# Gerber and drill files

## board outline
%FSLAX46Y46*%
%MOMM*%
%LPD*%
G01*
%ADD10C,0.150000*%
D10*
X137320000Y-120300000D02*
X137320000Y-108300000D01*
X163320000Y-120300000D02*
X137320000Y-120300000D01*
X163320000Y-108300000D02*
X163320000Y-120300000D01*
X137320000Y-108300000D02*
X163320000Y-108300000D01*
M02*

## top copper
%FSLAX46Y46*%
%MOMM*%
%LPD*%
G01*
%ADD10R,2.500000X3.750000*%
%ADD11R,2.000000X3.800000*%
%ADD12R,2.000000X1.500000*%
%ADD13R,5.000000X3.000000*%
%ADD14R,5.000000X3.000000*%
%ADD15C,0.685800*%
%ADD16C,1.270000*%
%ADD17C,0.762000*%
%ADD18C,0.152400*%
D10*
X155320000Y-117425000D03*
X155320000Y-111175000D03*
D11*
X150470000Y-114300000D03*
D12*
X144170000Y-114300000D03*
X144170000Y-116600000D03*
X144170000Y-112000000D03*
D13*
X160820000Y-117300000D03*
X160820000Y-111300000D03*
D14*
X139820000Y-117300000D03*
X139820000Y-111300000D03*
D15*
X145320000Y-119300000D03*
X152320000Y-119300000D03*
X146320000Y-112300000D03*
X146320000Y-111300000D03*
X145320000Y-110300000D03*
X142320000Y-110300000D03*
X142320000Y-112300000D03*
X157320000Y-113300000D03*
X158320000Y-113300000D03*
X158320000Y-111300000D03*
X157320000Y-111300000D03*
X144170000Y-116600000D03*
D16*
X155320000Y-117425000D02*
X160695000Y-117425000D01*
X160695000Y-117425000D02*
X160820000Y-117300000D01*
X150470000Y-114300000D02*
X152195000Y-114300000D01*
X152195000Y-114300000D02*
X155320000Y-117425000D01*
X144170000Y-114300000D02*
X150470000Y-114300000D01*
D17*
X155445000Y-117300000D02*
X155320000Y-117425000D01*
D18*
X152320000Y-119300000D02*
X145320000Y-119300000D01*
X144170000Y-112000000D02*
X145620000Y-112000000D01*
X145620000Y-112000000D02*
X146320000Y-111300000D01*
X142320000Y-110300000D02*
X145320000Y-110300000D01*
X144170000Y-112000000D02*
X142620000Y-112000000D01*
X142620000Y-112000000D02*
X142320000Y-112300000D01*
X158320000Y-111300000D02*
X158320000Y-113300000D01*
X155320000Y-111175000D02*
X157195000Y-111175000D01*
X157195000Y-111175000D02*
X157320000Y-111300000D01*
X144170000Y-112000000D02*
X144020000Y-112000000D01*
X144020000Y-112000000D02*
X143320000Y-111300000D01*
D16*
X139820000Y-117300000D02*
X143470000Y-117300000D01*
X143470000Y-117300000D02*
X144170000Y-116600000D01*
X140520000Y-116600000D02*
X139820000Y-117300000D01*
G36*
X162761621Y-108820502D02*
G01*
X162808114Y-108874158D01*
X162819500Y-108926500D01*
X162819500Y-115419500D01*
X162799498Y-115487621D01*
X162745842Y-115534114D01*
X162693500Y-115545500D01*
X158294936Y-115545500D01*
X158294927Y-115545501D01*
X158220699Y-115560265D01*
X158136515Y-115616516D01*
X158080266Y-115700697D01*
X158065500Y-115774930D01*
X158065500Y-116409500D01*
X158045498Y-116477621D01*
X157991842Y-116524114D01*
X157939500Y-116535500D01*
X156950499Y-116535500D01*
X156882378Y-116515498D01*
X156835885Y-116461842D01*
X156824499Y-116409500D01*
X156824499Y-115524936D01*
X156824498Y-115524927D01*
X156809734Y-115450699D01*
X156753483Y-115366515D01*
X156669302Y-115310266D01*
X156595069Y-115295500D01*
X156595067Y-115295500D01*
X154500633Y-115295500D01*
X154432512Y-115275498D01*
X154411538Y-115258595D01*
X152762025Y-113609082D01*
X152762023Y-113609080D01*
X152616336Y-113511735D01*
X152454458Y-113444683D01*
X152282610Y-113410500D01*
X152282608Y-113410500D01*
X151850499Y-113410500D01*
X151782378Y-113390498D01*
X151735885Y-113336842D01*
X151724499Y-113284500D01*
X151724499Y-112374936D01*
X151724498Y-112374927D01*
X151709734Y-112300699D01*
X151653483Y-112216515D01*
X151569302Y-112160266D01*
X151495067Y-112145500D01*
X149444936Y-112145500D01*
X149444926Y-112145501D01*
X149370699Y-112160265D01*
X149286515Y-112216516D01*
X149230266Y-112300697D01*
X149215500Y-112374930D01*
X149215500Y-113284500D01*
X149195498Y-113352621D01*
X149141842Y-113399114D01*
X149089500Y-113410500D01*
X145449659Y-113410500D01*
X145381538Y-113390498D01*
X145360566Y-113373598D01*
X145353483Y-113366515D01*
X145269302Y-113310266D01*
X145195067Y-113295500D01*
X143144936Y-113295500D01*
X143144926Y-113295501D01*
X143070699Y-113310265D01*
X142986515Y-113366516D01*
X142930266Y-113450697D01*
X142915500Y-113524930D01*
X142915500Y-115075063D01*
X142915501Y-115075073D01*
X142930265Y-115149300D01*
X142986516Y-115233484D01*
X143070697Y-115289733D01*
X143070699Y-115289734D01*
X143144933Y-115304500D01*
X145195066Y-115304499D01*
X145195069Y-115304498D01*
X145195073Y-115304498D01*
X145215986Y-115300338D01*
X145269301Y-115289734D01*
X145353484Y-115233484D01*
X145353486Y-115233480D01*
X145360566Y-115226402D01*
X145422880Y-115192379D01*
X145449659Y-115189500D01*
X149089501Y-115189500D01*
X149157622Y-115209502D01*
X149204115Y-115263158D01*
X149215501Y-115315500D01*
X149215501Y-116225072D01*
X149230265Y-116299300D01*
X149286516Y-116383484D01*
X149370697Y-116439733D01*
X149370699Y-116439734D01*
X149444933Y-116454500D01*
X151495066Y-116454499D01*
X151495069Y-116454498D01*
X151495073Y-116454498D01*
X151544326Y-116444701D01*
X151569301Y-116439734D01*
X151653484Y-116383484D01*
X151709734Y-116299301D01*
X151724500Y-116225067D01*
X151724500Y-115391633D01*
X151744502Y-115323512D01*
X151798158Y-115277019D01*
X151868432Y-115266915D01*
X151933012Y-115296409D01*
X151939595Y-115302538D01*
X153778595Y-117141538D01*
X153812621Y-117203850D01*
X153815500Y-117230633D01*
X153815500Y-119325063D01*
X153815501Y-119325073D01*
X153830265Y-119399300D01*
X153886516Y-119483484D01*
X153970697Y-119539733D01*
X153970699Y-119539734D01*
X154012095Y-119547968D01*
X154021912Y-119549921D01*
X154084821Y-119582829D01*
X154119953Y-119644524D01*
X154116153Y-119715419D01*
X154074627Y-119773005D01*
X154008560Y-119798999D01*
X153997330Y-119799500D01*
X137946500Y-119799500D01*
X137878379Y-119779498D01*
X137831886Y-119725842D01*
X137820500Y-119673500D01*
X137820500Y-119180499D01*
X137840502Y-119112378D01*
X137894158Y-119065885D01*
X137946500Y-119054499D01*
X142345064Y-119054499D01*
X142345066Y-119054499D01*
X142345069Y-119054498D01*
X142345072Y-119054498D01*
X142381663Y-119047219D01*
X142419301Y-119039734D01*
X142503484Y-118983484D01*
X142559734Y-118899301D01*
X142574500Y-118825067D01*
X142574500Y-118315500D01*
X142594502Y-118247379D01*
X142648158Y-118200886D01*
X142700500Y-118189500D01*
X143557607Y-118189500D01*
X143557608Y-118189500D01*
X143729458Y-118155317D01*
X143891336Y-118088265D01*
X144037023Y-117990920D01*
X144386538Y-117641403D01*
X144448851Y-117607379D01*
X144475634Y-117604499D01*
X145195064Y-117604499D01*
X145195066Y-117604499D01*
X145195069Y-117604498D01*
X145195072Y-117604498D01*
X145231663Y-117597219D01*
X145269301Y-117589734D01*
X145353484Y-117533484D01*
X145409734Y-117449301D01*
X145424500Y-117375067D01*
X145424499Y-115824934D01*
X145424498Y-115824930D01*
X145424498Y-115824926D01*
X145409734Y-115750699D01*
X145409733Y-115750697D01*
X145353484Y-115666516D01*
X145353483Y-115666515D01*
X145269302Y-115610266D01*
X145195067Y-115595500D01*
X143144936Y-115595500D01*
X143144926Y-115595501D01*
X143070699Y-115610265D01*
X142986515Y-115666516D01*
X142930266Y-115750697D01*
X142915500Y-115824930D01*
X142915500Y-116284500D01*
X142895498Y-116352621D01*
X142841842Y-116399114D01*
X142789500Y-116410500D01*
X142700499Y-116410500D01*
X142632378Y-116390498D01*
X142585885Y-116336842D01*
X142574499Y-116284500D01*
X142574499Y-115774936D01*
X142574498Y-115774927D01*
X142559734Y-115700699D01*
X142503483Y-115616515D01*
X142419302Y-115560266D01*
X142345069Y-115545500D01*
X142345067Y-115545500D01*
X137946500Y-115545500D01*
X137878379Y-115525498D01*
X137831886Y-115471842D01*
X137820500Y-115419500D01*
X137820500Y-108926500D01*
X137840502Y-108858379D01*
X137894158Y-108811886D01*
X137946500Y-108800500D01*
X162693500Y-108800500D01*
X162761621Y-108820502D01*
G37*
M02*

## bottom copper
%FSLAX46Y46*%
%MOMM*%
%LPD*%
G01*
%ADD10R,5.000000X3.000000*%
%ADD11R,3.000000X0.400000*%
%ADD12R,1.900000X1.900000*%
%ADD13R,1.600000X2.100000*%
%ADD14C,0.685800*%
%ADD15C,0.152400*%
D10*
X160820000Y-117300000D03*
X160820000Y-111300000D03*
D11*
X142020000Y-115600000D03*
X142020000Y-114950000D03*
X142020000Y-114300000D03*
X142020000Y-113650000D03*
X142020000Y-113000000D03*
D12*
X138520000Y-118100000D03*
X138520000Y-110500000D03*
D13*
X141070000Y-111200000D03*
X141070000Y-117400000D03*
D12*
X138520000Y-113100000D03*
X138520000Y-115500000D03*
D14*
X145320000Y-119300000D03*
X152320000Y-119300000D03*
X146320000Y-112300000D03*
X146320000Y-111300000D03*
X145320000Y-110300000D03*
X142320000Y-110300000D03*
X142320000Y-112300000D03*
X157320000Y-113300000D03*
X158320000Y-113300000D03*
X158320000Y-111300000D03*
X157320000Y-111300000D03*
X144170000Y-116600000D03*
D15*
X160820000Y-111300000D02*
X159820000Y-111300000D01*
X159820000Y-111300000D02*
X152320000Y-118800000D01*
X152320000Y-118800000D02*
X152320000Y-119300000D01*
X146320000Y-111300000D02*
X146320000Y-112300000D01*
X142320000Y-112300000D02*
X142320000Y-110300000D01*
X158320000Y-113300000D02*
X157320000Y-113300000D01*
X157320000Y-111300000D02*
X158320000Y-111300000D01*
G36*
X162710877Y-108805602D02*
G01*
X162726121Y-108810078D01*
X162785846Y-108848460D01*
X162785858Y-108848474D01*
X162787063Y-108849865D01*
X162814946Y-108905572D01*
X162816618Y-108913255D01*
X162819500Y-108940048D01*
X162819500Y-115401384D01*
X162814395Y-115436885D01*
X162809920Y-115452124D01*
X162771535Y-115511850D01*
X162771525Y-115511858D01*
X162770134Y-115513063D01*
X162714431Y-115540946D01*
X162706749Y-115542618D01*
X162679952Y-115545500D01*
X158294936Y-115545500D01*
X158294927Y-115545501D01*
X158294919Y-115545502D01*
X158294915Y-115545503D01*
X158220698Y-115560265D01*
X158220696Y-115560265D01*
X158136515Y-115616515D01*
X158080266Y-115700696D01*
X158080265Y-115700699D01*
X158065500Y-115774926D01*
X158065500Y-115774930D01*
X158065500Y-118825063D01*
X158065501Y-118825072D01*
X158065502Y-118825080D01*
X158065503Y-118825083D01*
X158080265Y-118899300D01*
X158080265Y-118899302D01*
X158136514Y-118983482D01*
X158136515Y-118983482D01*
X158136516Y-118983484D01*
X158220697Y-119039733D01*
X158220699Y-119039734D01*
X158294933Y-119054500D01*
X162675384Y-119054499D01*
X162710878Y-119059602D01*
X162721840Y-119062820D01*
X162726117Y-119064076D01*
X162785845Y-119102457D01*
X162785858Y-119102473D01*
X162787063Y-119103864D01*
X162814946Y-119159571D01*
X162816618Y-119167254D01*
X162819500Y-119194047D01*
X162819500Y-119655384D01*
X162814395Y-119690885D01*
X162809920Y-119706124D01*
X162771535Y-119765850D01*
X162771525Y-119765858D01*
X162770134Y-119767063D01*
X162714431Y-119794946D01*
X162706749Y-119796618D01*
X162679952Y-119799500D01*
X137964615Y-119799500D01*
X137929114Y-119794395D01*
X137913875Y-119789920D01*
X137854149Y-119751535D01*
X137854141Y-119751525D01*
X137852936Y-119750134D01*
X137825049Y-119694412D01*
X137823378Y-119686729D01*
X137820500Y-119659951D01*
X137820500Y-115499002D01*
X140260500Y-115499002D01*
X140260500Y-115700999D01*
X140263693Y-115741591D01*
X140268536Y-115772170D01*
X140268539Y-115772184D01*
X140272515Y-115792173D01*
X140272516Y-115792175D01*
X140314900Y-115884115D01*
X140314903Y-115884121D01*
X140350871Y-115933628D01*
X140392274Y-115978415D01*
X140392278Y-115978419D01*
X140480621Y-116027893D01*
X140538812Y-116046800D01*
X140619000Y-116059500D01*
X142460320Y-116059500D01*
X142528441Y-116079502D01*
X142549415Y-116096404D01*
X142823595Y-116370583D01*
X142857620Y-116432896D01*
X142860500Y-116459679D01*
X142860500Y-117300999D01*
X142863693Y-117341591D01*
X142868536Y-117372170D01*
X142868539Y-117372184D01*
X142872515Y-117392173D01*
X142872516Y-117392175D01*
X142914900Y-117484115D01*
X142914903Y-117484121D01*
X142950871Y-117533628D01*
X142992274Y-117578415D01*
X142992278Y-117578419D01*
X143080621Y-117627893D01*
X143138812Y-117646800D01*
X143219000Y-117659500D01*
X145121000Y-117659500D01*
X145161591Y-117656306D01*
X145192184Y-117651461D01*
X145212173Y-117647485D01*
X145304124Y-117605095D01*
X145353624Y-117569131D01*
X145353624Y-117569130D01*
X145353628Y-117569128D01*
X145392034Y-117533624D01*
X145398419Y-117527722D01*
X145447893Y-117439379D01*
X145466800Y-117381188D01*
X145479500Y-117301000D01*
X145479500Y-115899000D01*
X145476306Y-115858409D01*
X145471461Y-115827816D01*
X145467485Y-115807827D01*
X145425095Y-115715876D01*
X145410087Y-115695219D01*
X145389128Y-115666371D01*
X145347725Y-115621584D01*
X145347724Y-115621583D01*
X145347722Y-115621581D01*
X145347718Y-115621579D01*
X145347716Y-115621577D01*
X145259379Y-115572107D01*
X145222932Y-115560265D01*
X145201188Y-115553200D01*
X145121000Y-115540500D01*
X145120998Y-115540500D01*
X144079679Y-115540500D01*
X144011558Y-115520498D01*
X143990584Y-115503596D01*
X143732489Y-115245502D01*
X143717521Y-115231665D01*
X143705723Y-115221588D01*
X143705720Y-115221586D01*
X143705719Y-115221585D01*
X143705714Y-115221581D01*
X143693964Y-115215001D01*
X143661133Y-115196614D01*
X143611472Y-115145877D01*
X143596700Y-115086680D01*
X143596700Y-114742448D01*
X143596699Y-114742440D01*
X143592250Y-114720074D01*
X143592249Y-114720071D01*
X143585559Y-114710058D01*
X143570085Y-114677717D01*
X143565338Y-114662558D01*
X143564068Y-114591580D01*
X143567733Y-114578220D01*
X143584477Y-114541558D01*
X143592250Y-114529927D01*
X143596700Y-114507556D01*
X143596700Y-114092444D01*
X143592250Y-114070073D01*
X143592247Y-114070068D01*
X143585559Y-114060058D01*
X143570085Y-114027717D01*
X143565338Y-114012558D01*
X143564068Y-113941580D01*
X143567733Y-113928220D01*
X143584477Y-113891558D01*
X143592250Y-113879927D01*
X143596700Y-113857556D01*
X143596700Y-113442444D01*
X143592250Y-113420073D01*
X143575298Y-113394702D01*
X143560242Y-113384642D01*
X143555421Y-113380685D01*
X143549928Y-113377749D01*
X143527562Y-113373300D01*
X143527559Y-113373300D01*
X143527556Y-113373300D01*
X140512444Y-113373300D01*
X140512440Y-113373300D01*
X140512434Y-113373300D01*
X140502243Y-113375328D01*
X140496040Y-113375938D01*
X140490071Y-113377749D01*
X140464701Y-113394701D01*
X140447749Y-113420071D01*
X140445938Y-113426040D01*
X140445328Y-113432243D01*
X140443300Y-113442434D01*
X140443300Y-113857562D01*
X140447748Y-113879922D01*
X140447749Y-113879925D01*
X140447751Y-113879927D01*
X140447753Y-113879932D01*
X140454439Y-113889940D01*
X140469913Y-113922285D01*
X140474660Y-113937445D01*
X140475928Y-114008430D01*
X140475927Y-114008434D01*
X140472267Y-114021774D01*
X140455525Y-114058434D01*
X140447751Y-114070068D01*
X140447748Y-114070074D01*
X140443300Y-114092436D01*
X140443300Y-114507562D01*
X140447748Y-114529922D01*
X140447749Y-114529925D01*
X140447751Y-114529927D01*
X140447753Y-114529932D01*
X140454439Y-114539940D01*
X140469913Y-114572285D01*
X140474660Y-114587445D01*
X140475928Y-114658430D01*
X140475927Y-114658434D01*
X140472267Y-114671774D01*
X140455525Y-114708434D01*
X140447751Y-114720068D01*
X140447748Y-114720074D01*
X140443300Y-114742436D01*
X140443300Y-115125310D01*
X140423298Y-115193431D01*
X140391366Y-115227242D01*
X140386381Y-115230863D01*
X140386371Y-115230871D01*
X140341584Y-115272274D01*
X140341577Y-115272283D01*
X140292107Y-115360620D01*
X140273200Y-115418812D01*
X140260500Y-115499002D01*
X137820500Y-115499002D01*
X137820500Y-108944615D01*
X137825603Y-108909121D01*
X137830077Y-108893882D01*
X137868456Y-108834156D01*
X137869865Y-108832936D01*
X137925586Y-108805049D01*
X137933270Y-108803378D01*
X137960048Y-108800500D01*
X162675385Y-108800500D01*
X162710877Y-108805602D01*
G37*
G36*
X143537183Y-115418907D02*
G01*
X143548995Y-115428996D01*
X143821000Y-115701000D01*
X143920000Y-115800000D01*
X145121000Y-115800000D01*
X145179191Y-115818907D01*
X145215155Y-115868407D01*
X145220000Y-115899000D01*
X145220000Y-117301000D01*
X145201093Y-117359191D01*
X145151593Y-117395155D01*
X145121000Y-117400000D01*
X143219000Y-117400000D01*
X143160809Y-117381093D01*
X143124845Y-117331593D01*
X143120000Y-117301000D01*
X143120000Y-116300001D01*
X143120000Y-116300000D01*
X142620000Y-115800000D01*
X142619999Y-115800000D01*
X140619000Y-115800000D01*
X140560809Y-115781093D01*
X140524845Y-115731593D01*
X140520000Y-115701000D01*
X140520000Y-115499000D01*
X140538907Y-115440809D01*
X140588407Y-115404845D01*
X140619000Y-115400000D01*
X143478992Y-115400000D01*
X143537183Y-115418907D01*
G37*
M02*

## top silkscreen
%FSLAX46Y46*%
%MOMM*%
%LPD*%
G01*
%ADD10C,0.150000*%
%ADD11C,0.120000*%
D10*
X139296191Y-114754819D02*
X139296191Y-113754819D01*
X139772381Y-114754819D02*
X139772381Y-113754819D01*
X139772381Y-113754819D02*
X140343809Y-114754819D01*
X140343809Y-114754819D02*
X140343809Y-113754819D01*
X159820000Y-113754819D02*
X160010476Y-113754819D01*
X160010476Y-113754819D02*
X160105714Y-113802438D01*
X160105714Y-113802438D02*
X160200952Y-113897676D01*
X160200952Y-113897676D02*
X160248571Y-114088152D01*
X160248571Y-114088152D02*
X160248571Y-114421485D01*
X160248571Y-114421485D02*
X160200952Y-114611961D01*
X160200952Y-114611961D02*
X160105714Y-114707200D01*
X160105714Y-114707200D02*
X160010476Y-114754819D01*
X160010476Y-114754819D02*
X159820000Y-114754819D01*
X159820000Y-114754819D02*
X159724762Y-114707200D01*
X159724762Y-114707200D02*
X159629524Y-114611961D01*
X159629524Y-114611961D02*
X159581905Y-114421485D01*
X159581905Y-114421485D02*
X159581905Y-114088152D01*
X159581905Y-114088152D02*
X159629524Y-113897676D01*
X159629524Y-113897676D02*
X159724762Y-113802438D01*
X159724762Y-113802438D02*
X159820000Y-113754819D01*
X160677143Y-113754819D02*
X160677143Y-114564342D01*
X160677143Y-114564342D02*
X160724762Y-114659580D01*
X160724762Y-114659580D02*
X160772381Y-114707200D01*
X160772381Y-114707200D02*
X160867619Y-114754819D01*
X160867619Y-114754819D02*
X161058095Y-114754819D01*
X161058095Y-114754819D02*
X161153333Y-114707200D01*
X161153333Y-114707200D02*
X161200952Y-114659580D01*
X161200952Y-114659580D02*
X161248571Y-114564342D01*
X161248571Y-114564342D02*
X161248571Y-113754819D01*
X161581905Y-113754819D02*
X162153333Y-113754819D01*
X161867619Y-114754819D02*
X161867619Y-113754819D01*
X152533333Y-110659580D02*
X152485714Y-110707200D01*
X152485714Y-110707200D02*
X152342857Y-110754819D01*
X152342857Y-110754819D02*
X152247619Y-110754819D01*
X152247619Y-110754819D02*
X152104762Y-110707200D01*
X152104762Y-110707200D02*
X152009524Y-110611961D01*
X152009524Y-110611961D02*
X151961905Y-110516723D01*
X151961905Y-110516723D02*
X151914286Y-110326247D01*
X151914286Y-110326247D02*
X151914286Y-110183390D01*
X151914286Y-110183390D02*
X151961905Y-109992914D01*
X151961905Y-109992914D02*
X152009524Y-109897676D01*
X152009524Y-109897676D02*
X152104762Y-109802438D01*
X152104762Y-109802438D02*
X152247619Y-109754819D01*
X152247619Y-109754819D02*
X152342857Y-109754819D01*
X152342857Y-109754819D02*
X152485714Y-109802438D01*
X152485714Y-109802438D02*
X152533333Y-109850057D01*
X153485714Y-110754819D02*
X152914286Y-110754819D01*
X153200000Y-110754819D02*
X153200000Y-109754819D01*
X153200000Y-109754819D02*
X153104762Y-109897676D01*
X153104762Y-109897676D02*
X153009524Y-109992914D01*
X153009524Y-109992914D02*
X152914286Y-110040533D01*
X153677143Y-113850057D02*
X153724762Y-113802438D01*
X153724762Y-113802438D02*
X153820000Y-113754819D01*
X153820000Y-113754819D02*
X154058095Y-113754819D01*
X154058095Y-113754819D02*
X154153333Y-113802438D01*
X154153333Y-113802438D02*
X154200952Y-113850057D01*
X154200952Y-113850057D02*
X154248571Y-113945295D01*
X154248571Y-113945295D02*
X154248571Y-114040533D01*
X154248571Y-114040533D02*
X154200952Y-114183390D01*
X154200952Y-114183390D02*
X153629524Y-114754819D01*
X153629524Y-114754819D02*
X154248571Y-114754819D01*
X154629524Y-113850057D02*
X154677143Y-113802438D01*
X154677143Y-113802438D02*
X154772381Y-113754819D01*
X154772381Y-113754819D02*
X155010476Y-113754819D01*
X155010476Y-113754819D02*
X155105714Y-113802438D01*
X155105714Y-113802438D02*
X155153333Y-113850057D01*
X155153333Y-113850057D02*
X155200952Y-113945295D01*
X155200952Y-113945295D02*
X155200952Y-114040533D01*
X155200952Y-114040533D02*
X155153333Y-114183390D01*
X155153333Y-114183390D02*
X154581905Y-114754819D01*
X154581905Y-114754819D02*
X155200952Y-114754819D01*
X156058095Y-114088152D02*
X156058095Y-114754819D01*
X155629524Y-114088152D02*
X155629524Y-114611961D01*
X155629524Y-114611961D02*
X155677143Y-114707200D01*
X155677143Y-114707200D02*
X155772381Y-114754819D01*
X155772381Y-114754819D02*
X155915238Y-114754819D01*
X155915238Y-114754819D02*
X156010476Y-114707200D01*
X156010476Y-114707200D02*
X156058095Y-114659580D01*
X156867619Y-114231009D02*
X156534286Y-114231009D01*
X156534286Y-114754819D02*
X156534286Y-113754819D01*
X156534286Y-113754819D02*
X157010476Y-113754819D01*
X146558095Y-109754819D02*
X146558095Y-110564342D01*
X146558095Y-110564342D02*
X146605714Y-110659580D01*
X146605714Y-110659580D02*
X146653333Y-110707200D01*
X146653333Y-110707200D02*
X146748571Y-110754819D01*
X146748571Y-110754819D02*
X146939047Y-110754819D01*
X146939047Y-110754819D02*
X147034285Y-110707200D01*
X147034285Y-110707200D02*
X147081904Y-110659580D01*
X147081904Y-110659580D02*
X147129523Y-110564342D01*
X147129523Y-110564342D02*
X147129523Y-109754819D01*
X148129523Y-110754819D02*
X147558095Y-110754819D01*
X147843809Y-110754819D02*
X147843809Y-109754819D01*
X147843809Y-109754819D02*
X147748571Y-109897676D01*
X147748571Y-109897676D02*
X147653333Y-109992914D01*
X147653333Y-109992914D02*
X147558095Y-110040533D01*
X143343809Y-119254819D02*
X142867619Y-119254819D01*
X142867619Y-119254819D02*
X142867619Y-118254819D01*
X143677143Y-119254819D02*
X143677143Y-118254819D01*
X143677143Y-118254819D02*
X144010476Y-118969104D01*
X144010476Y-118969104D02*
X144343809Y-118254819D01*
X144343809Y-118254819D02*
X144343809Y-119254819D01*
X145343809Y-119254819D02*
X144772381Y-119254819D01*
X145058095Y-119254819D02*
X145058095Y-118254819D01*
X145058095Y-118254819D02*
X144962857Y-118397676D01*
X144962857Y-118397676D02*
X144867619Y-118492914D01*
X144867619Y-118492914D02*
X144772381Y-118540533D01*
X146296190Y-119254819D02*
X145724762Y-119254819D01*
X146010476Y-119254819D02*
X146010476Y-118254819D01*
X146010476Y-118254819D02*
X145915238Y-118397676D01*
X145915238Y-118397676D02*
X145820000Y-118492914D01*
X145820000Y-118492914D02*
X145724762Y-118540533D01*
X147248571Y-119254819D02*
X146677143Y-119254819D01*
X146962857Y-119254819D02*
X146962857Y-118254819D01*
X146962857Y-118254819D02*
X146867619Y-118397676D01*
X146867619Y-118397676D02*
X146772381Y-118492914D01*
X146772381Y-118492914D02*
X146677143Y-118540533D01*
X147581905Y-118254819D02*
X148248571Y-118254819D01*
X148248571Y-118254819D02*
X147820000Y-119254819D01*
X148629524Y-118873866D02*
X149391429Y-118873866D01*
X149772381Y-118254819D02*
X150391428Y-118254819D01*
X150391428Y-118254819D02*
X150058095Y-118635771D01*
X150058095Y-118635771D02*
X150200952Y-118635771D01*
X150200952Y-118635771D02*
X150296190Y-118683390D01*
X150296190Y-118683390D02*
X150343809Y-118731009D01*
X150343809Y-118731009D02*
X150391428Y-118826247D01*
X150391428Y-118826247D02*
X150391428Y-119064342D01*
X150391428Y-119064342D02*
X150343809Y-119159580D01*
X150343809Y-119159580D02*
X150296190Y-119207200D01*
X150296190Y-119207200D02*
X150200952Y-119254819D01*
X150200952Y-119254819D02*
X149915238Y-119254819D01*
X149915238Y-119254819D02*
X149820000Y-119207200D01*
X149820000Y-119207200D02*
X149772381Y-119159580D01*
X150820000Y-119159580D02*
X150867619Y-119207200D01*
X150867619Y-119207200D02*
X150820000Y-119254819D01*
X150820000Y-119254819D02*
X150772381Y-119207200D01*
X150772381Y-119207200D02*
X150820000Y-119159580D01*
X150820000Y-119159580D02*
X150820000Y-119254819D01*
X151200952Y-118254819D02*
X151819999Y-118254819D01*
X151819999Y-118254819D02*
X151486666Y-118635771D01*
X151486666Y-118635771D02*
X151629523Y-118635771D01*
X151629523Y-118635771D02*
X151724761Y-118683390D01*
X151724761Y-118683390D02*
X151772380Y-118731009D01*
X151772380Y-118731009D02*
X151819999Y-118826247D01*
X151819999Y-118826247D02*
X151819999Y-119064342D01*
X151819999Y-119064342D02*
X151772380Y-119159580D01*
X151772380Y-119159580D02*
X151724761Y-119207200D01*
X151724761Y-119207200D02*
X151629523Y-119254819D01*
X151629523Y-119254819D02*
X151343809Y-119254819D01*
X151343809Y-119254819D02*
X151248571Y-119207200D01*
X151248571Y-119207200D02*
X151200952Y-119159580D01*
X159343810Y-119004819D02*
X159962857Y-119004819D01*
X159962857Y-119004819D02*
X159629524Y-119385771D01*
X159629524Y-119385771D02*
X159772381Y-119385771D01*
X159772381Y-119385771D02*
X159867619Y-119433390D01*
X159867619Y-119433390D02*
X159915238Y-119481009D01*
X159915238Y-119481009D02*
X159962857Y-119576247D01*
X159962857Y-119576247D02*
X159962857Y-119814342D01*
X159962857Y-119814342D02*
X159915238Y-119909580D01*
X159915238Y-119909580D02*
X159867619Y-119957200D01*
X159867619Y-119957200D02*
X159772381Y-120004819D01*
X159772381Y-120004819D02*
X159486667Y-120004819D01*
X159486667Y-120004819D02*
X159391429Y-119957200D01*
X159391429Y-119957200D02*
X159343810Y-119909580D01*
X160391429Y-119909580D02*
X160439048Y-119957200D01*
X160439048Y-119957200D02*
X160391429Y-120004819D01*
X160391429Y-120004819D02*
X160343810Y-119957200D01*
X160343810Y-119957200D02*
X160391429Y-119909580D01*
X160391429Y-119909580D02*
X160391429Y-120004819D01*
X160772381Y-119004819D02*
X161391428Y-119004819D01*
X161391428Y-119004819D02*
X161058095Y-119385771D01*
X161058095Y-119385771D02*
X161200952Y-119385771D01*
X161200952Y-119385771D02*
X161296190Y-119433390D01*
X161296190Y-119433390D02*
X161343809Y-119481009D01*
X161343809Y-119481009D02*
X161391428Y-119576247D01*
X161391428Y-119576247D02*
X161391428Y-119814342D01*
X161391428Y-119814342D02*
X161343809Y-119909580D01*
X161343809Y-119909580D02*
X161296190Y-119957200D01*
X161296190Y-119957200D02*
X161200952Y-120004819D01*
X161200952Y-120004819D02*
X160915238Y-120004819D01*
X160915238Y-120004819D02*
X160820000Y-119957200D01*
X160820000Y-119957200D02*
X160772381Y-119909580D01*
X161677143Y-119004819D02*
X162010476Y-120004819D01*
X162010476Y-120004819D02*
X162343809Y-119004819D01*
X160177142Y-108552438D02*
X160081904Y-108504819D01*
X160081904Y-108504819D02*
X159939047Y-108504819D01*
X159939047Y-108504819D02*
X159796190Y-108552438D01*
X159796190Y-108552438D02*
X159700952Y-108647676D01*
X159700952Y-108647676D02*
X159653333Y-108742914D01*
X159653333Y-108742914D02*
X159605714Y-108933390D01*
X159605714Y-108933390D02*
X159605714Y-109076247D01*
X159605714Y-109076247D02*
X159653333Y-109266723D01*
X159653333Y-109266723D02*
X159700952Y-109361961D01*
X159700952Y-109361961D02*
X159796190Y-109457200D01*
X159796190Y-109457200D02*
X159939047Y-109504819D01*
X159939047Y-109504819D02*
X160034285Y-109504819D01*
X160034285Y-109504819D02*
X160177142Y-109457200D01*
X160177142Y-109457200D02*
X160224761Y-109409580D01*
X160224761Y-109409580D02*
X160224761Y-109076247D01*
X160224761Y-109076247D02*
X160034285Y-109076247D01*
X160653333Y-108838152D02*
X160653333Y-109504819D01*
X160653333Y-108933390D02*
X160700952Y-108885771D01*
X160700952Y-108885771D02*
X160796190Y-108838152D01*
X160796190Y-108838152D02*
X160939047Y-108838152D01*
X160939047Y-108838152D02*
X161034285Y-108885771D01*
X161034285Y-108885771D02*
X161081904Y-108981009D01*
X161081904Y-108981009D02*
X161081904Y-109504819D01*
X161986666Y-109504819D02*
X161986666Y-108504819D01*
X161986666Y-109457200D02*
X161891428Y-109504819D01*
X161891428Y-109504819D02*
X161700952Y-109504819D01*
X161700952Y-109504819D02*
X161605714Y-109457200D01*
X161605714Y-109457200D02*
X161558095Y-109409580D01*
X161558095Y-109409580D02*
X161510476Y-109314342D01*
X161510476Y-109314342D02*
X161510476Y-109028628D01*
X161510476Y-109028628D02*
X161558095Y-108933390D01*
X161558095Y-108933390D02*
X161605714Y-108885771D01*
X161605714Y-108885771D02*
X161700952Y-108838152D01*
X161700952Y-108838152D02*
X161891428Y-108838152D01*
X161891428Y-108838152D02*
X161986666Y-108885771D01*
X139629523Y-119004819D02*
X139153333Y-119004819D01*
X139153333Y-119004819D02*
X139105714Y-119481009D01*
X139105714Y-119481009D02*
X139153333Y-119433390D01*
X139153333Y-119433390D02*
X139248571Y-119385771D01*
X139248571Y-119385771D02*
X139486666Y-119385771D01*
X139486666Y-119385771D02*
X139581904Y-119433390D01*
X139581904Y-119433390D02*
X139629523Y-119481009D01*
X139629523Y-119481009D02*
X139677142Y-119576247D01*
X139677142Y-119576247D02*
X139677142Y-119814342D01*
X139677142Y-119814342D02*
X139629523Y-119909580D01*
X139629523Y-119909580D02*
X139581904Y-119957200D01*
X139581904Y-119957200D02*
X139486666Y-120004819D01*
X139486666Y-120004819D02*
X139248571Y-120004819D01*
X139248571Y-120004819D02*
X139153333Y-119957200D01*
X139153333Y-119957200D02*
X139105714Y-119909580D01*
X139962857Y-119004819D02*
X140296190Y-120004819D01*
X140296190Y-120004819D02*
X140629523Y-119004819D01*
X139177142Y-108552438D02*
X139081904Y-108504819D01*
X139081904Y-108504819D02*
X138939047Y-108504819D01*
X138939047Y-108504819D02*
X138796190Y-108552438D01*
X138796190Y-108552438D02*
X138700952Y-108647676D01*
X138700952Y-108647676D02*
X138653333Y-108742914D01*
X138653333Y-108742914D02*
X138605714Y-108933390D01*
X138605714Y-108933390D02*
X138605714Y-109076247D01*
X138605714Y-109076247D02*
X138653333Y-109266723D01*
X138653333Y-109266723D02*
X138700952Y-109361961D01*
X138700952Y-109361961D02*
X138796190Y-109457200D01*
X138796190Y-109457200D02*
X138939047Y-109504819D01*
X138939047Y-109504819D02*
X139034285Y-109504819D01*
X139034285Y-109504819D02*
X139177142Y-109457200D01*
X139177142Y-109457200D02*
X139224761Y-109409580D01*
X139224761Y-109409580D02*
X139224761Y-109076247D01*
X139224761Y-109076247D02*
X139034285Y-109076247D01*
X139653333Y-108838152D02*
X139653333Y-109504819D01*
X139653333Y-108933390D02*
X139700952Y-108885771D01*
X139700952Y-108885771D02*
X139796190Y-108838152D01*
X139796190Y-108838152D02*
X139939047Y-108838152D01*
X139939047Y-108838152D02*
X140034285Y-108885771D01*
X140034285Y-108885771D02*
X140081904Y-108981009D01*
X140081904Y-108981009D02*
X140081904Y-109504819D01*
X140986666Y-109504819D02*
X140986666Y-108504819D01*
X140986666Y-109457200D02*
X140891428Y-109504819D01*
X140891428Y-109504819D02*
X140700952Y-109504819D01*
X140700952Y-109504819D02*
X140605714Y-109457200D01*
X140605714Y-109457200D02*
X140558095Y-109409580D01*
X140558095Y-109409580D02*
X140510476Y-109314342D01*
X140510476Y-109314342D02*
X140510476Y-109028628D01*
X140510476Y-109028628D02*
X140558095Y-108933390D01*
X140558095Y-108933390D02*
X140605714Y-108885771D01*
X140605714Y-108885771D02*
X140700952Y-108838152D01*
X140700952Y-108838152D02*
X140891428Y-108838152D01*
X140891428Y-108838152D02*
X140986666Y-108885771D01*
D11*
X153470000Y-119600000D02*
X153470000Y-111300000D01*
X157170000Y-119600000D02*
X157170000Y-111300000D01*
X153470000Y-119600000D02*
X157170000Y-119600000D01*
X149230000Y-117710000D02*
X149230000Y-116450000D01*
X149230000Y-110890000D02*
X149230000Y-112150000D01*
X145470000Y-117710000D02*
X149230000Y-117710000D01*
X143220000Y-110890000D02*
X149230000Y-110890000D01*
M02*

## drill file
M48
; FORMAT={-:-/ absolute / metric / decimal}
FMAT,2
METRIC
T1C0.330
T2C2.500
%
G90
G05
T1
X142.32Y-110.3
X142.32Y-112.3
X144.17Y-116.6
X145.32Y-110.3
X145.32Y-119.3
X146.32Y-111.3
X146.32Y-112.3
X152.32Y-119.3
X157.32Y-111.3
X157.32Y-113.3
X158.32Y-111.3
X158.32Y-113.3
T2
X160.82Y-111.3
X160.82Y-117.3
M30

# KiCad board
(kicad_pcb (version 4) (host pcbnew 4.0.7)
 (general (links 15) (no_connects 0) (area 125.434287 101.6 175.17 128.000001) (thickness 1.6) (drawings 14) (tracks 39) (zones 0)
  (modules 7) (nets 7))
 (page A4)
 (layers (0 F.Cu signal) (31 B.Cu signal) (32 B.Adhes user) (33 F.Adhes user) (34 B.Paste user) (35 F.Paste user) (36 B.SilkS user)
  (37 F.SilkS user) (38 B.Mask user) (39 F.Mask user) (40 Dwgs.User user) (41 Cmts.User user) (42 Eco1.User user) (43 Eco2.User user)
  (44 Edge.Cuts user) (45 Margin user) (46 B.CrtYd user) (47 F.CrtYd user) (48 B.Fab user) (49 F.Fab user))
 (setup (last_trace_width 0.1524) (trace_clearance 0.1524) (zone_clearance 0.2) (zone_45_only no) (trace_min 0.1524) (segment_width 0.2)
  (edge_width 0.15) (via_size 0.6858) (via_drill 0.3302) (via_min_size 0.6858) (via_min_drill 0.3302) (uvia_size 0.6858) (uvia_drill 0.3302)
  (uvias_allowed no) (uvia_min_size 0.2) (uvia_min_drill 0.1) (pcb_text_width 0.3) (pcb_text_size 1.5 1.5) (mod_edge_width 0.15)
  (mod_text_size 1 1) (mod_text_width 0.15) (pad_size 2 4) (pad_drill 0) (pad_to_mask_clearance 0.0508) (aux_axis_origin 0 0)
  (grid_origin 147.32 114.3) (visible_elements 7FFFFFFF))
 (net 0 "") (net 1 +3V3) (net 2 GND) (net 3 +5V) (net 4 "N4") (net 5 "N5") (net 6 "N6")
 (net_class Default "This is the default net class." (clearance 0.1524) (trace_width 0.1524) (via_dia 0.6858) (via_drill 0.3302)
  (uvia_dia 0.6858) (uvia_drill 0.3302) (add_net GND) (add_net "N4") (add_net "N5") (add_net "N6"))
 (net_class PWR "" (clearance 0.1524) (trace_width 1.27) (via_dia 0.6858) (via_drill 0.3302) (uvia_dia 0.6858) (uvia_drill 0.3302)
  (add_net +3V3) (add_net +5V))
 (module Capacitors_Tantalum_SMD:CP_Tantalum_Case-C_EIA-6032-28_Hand (layer F.Cu) (at 155.32 114.3 90)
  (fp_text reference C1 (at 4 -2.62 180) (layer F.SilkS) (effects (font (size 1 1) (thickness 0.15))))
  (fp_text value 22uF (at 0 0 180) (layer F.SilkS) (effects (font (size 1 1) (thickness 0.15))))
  (fp_line (start -5.3 -1.85) (end 3 -1.85) (layer F.SilkS) (width 0.12))
  (fp_line (start -5.3 1.85) (end 3 1.85) (layer F.SilkS) (width 0.12))
  (fp_line (start -5.3 -1.85) (end -5.3 1.85) (layer F.SilkS) (width 0.12))
  (pad 1 smd rect (at -3.125 0 90) (size 3.75 2.5) (layers F.Cu F.Paste F.Mask) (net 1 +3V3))
  (pad 2 smd rect (at 3.125 0 90) (size 3.75 2.5) (layers F.Cu F.Paste F.Mask) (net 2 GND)))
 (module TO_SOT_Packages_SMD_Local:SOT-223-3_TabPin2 (layer F.Cu) (at 147.32 114.3)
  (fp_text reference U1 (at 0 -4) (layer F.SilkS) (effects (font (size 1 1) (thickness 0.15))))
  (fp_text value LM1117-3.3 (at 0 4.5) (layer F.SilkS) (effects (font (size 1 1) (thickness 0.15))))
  (fp_line (start 1.91 3.41) (end 1.91 2.15) (layer F.SilkS) (width 0.12))
  (fp_line (start 1.91 -3.41) (end 1.91 -2.15) (layer F.SilkS) (width 0.12))
  (fp_line (start -1.85 3.41) (end 1.91 3.41) (layer F.SilkS) (width 0.12))
  (fp_line (start -4.1 -3.41) (end 1.91 -3.41) (layer F.SilkS) (width 0.12))
  (pad 2 smd rect (at 3.15 0) (size 2 3.8) (layers F.Cu F.Paste F.Mask) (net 1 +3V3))
  (pad 2 smd rect (at -3.15 0) (size 2 1.5) (layers F.Cu F.Paste F.Mask) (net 1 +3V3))
  (pad 3 smd rect (at -3.15 2.3) (size 2 1.5) (layers F.Cu F.Paste F.Mask) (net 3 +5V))
  (pad 1 smd rect (at -3.15 -2.3) (size 2 1.5) (layers F.Cu F.Paste F.Mask) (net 2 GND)))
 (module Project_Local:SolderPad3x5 (layer F.Cu) (at 160.82 117.3)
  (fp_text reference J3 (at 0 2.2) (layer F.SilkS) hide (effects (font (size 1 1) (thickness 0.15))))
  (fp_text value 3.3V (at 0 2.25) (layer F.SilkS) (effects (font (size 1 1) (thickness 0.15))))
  (pad 1 thru_hole rect (at 0 0 90) (size 3 5) (drill 2.5) (layers *.Cu *.Mask) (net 1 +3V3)))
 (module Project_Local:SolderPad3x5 (layer F.Cu) (at 160.82 111.3)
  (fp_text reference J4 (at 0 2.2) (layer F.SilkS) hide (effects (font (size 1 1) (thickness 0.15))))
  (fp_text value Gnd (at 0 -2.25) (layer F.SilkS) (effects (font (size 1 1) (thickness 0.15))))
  (pad 1 thru_hole rect (at 0 0 90) (size 3 5) (drill 2.5) (layers *.Cu *.Mask) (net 2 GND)))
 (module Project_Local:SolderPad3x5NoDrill (layer F.Cu) (at 139.82 117.3)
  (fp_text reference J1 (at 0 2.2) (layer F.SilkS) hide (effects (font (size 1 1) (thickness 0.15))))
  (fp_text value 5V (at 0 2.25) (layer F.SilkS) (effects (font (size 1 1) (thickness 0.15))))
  (pad 1 connect rect (at 0 0 90) (size 3 5) (layers F.Cu F.Mask) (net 3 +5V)))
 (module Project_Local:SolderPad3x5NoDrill (layer F.Cu) (at 139.82 111.3)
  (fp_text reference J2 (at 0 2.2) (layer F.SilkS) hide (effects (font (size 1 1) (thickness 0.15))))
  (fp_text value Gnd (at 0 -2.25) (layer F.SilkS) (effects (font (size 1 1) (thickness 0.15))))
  (pad 1 connect rect (at 0 0 90) (size 3 5) (layers F.Cu F.Mask) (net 2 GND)))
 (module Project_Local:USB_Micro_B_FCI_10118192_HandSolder (layer B.Cu) (at 138.52 114.3)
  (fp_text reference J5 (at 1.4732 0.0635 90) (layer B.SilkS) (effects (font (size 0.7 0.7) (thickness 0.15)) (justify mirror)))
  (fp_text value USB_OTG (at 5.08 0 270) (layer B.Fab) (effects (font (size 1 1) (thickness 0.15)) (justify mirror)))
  (pad 1 smd rect (at 3.5 1.3) (size 3 0.4) (layers B.Cu B.Paste B.Mask) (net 3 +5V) (solder_mask_margin 0.0762)
   (solder_paste_margin -0.0762) (clearance 0.0762))
  (pad 2 smd rect (at 3.5 0.65) (size 3 0.4) (layers B.Cu B.Paste B.Mask) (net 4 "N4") (solder_mask_margin 0.0762)
   (solder_paste_margin -0.0762) (clearance 0.0762))
  (pad 3 smd rect (at 3.5 0) (size 3 0.4) (layers B.Cu B.Paste B.Mask) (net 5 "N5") (solder_mask_margin 0.0762)
   (solder_paste_margin -0.0762) (clearance 0.0762))
  (pad 4 smd rect (at 3.5 -0.65) (size 3 0.4) (layers B.Cu B.Paste B.Mask) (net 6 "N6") (solder_mask_margin 0.0762)
   (solder_paste_margin -0.0762) (clearance 0.0762))
  (pad 5 smd rect (at 3.5 -1.3) (size 3 0.4) (layers B.Cu B.Paste B.Mask) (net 2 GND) (solder_mask_margin 0.0762)
   (solder_paste_margin -0.0762) (clearance 0.0762))
  (pad 6 smd rect (at 0 3.8) (size 1.9 1.9) (layers B.Cu B.Paste B.Mask) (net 2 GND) (solder_mask_margin 0.0762)
   (solder_paste_margin -0.0762) (clearance 0.0762))
  (pad 6 smd rect (at 0 -3.8) (size 1.9 1.9) (layers B.Cu B.Paste B.Mask) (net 2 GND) (solder_mask_margin 0.0762)
   (solder_paste_margin -0.0762) (clearance 0.0762))
  (pad 6 smd rect (at 2.55 -3.1) (size 1.6 2.1) (layers B.Cu B.Paste B.Mask) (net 2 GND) (solder_mask_margin 0.0762)
   (solder_paste_margin -0.0762) (clearance 0.0762))
  (pad 6 smd rect (at 2.55 3.1) (size 1.6 2.1) (layers B.Cu B.Paste B.Mask) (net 2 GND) (solder_mask_margin 0.0762) (clearance 0.0762))
  (pad 6 smd rect (at 0 -1.2) (size 1.9 1.9) (layers B.Cu B.Paste B.Mask) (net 2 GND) (solder_mask_margin 0.0762)
   (solder_paste_margin -0.0762) (clearance 0.0762))
  (pad 6 smd rect (at 0 1.2) (size 1.9 1.9) (layers B.Cu B.Paste B.Mask) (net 2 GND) (solder_mask_margin 0.0762)
   (solder_paste_margin -0.0762) (clearance 0.0762)))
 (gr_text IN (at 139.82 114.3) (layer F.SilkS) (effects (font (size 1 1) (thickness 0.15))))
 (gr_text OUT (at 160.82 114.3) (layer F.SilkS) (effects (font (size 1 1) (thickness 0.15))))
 (gr_line (start 137.32 120.3) (end 137.32 108.3) (layer Edge.Cuts) (width 0.15))
 (gr_line (start 163.32 120.3) (end 137.32 120.3) (layer Edge.Cuts) (width 0.15))
 (gr_line (start 163.32 108.3) (end 163.32 120.3) (layer Edge.Cuts) (width 0.15))
 (gr_line (start 137.32 108.3) (end 163.32 108.3) (layer Edge.Cuts) (width 0.15))
 (segment (start 155.32 117.425) (end 160.695 117.425) (width 1.27) (layer F.Cu) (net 1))
 (segment (start 160.695 117.425) (end 160.82 117.3) (width 1.27) (layer F.Cu) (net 1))
 (segment (start 150.47 114.3) (end 152.195 114.3) (width 1.27) (layer F.Cu) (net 1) (status 10))
 (segment (start 152.195 114.3) (end 155.32 117.425) (width 1.27) (layer F.Cu) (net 1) (status 20))
 (segment (start 144.17 114.3) (end 150.47 114.3) (width 1.27) (layer F.Cu) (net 1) (status 30))
 (segment (start 155.445 117.3) (end 155.32 117.425) (width 0.762) (layer F.Cu) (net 1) (status 30))
 (segment (start 152.32 119.3) (end 145.32 119.3) (width 0.1524) (layer F.Cu) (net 2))
 (via (at 145.32 119.3) (size 0.6858) (drill 0.3302) (layers F.Cu B.Cu) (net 2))
 (segment (start 160.82 111.3) (end 159.82 111.3) (width 0.1524) (layer B.Cu) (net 2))
 (segment (start 159.82 111.3) (end 152.32 118.8) (width 0.1524) (layer B.Cu) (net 2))
 (segment (start 152.32 118.8) (end 152.32 119.3) (width 0.1524) (layer B.Cu) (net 2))
 (via (at 152.32 119.3) (size 0.6858) (drill 0.3302) (layers F.Cu B.Cu) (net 2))
 (segment (start 146.32 111.3) (end 146.32 112.3) (width 0.1524) (layer B.Cu) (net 2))
 (via (at 146.32 112.3) (size 0.6858) (drill 0.3302) (layers F.Cu B.Cu) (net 2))
 (segment (start 144.17 112) (end 145.62 112) (width 0.1524) (layer F.Cu) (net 2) (status 10))
 (segment (start 145.62 112) (end 146.32 111.3) (width 0.1524) (layer F.Cu) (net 2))
 (via (at 146.32 111.3) (size 0.6858) (drill 0.3302) (layers F.Cu B.Cu) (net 2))
 (segment (start 142.32 110.3) (end 145.32 110.3) (width 0.1524) (layer F.Cu) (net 2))
 (via (at 145.32 110.3) (size 0.6858) (drill 0.3302) (layers F.Cu B.Cu) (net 2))
 (segment (start 142.32 112.3) (end 142.32 110.3) (width 0.1524) (layer B.Cu) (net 2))
 (via (at 142.32 110.3) (size 0.6858) (drill 0.3302) (layers F.Cu B.Cu) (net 2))
 (segment (start 144.17 112) (end 142.62 112) (width 0.1524) (layer F.Cu) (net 2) (status 10))
 (segment (start 142.62 112) (end 142.32 112.3) (width 0.1524) (layer F.Cu) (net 2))
 (via (at 142.32 112.3) (size 0.6858) (drill 0.3302) (layers F.Cu B.Cu) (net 2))
 (segment (start 158.32 113.3) (end 157.32 113.3) (width 0.1524) (layer B.Cu) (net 2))
 (via (at 157.32 113.3) (size 0.6858) (drill 0.3302) (layers F.Cu B.Cu) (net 2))
 (segment (start 158.32 111.3) (end 158.32 113.3) (width 0.1524) (layer F.Cu) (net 2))
 (via (at 158.32 113.3) (size 0.6858) (drill 0.3302) (layers F.Cu B.Cu) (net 2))
 (segment (start 157.32 111.3) (end 158.32 111.3) (width 0.1524) (layer B.Cu) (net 2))
 (via (at 158.32 111.3) (size 0.6858) (drill 0.3302) (layers F.Cu B.Cu) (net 2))
 (segment (start 155.32 111.175) (end 157.195 111.175) (width 0.1524) (layer F.Cu) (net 2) (status 10))
 (segment (start 157.195 111.175) (end 157.32 111.3) (width 0.1524) (layer F.Cu) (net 2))
 (via (at 157.32 111.3) (size 0.6858) (drill 0.3302) (layers F.Cu B.Cu) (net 2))
 (segment (start 144.17 112) (end 144.02 112) (width 0.1524) (layer F.Cu) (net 2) (status 30))
 (segment (start 144.02 112) (end 143.32 111.3) (width 0.1524) (layer F.Cu) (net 2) (status 30))
 (segment (start 139.82 117.3) (end 143.47 117.3) (width 1.27) (layer F.Cu) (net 3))
 (segment (start 143.47 117.3) (end 144.17 116.6) (width 1.27) (layer F.Cu) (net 3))
 (via (at 144.17 116.6) (size 0.6858) (drill 0.3302) (layers F.Cu B.Cu) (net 3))
 (segment (start 140.52 116.6) (end 139.82 117.3) (width 1.27) (layer F.Cu) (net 3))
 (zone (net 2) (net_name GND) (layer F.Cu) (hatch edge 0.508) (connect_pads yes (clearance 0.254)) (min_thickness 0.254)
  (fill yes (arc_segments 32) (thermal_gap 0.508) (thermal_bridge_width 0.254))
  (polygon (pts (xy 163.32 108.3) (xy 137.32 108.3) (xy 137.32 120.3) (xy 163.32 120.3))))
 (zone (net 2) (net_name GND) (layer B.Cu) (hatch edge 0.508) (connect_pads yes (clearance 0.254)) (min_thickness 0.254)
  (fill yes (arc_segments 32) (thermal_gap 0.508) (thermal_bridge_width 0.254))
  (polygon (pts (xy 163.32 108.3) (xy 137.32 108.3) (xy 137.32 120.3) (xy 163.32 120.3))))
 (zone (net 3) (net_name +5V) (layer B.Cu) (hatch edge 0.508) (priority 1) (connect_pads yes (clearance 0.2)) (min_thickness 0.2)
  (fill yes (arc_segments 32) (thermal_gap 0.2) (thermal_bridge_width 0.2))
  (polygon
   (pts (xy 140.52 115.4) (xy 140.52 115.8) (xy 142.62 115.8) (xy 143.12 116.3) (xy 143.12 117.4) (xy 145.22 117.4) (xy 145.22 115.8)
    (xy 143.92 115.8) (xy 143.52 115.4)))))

